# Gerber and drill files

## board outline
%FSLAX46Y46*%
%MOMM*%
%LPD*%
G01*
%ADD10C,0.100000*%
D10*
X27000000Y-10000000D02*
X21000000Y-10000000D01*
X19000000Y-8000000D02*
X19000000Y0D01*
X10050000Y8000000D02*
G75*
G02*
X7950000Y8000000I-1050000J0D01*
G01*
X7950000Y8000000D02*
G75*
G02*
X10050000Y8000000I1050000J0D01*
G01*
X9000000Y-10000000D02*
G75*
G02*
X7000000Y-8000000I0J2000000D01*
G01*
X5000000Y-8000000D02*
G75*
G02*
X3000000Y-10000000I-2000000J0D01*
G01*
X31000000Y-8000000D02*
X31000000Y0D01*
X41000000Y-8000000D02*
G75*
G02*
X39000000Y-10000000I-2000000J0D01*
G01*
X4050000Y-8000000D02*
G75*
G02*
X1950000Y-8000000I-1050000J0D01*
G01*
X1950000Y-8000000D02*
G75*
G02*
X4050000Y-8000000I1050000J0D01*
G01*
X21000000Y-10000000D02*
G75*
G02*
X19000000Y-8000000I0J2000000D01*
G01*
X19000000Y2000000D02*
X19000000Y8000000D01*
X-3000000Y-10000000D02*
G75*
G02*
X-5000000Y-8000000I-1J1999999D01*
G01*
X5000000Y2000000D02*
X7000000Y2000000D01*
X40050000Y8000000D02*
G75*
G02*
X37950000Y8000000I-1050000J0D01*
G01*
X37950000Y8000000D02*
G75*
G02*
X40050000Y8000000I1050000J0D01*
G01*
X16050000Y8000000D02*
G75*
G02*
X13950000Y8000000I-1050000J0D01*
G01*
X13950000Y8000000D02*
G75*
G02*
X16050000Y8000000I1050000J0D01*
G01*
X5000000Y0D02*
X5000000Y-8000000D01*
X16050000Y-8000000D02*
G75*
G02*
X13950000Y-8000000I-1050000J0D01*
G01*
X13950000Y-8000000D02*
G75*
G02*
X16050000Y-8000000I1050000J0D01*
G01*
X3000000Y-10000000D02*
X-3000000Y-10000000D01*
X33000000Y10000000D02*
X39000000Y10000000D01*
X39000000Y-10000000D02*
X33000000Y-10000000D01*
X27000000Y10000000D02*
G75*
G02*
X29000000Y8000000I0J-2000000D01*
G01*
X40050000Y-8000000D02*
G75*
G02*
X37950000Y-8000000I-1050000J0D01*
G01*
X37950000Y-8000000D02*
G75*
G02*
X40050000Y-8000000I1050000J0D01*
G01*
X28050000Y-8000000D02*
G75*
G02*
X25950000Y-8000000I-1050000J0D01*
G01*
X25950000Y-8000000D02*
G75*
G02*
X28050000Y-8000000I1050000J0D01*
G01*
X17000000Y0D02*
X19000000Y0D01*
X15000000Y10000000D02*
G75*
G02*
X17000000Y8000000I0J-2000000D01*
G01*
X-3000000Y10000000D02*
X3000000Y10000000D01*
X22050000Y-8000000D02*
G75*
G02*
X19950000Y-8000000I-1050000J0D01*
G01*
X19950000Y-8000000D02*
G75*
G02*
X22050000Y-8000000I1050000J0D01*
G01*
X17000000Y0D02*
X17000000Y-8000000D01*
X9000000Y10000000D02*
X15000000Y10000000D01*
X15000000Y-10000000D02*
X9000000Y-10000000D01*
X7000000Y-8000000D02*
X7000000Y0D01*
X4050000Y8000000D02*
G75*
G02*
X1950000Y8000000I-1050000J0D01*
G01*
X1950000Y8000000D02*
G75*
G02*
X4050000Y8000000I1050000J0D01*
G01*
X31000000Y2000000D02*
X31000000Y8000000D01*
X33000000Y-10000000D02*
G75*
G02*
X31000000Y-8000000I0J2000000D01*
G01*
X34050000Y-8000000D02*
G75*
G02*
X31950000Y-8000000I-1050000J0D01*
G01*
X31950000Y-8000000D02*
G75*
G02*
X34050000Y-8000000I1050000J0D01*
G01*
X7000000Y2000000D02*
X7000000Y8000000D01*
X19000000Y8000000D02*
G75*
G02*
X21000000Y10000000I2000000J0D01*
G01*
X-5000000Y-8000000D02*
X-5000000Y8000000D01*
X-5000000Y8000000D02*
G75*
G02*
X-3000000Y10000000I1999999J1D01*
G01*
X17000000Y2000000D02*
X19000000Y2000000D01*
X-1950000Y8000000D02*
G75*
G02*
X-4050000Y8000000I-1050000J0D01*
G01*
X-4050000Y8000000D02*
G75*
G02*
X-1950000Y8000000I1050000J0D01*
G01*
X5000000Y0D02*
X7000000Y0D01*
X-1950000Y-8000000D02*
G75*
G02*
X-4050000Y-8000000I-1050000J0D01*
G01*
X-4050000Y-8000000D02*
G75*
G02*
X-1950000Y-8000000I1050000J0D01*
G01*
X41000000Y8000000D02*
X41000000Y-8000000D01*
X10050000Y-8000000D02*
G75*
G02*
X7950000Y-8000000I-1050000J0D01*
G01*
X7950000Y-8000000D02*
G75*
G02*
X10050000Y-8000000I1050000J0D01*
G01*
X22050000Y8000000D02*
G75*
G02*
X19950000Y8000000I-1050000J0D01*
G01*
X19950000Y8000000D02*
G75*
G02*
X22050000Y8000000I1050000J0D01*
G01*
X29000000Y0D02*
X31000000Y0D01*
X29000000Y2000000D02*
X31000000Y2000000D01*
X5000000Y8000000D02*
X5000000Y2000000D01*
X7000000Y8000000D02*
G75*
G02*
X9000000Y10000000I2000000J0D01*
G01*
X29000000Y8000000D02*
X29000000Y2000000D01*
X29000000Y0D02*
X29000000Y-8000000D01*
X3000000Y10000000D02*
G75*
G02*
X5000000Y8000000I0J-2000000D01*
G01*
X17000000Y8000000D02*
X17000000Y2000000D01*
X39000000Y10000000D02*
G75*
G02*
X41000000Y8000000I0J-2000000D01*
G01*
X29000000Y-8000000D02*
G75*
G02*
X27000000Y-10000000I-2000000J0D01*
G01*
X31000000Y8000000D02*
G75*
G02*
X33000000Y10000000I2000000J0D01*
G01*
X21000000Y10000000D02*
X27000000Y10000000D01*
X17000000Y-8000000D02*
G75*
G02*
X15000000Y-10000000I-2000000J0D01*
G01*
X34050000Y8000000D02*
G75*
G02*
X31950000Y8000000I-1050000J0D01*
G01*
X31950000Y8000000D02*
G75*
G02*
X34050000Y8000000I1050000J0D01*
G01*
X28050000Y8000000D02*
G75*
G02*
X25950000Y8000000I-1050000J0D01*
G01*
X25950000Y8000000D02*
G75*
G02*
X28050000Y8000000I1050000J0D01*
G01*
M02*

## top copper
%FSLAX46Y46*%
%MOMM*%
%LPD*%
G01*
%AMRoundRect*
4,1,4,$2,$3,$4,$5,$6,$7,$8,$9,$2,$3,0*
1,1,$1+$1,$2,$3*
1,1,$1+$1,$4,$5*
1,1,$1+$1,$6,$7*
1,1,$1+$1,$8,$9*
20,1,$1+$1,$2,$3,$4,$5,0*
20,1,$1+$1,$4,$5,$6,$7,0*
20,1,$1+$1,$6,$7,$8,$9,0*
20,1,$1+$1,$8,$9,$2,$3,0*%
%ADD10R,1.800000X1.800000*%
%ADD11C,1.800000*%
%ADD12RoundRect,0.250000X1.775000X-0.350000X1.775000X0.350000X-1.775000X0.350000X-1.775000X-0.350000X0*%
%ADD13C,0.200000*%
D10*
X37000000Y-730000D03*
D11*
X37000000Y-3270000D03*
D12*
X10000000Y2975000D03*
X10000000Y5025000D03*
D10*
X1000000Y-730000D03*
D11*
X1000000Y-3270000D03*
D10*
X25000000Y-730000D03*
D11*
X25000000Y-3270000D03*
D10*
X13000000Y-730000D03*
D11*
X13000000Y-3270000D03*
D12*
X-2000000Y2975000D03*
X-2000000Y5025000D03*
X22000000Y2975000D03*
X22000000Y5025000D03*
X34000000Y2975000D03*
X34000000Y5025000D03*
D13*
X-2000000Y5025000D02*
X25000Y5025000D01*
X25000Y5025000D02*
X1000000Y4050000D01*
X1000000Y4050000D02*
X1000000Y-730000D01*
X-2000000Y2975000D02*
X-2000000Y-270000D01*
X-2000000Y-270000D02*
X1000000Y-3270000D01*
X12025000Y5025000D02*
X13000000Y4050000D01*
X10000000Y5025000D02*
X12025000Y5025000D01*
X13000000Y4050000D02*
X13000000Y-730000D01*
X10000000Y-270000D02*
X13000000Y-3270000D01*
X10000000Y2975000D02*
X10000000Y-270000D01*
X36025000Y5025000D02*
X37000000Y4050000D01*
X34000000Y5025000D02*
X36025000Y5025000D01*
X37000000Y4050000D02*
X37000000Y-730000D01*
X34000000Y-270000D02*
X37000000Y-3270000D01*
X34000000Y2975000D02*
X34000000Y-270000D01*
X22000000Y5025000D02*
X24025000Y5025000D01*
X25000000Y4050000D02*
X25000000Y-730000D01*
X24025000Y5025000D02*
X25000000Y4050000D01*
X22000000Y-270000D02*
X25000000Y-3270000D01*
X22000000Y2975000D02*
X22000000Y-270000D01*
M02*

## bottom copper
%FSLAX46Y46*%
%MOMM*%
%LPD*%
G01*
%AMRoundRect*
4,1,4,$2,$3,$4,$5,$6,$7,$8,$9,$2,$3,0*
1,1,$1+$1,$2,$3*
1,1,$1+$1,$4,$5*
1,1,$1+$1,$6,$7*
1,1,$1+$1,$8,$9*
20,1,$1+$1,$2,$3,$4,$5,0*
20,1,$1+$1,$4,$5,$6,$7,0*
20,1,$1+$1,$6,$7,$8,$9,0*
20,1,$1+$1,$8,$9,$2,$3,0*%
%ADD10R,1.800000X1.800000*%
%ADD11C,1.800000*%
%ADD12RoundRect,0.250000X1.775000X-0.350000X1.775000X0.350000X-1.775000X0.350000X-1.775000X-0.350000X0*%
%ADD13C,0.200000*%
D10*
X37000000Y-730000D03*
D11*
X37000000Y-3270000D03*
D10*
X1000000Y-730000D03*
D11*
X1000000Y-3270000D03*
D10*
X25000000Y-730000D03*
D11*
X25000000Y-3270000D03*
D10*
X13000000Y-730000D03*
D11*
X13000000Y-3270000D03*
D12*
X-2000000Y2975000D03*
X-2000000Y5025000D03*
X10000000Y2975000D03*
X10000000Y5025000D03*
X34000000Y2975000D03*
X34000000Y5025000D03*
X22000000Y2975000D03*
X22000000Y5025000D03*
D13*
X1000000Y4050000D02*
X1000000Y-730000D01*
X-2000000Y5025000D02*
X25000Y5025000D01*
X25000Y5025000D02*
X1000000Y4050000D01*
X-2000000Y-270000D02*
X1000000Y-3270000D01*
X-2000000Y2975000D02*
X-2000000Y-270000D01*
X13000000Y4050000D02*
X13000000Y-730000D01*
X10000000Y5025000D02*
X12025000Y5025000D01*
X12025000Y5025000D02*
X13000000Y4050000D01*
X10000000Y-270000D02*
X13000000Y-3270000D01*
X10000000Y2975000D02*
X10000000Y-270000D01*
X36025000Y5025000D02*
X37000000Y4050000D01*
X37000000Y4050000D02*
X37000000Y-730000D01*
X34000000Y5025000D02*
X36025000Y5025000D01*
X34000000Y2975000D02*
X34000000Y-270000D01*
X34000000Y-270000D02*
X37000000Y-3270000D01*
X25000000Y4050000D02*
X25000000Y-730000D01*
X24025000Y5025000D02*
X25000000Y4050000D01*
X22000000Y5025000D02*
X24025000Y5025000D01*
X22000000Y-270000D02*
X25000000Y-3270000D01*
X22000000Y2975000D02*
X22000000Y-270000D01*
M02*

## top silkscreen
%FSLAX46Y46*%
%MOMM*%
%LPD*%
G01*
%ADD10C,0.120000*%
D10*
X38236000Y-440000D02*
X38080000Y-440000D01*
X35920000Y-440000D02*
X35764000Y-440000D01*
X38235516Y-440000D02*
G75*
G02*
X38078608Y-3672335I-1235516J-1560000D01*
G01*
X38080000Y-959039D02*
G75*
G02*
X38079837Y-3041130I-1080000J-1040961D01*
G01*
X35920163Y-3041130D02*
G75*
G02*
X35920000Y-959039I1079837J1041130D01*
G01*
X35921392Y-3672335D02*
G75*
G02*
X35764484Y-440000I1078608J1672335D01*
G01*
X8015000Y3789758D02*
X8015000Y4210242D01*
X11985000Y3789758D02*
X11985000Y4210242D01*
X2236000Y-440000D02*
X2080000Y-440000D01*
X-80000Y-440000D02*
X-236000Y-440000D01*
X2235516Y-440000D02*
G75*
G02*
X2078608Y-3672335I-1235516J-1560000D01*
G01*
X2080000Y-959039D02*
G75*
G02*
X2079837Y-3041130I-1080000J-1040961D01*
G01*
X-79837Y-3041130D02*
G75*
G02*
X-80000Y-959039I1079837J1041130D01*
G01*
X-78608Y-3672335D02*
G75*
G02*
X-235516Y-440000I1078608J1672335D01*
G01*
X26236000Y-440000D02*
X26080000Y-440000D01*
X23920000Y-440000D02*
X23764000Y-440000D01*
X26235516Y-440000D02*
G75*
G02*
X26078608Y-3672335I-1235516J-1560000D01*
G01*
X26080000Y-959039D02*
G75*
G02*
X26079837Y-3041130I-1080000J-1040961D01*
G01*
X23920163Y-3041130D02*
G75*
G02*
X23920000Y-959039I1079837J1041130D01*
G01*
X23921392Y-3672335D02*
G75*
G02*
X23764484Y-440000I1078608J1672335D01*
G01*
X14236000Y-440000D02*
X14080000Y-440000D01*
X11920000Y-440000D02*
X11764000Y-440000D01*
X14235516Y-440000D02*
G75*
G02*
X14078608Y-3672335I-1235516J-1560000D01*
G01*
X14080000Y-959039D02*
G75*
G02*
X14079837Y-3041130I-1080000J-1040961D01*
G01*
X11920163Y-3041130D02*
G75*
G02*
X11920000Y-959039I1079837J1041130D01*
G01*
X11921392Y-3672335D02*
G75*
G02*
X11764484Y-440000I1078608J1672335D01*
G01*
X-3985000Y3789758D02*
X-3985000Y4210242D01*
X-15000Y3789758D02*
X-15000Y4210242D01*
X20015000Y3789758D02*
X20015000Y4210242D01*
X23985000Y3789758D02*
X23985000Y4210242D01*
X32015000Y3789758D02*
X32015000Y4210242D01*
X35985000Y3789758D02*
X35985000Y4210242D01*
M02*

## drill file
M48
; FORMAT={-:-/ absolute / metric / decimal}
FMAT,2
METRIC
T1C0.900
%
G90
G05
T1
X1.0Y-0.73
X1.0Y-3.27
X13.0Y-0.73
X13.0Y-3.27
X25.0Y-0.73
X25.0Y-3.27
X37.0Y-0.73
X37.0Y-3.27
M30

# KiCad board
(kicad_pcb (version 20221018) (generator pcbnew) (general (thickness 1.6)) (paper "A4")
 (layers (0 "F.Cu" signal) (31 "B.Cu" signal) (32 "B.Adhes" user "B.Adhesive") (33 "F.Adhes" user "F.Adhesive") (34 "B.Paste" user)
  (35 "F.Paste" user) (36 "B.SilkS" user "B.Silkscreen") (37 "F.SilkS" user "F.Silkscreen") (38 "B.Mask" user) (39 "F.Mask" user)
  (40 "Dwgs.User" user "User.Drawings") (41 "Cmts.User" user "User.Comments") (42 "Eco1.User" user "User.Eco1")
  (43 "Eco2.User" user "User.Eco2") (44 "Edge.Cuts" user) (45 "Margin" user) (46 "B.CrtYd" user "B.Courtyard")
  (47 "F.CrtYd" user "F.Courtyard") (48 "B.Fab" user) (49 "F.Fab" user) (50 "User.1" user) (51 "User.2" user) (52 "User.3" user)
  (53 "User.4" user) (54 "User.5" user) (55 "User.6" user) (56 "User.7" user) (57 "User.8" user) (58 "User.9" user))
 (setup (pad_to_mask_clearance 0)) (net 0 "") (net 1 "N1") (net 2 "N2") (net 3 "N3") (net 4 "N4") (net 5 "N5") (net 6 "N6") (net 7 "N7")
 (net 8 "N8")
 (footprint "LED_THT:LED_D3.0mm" (layer "F.Cu") (at 37 0.73 -90)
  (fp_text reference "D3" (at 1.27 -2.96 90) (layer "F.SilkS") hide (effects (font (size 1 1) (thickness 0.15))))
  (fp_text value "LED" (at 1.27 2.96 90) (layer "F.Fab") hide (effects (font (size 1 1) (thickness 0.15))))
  (fp_line (start -0.29 -1.236) (end -0.29 -1.08) (stroke (width 0.12) (type solid)) (layer "F.SilkS"))
  (fp_line (start -0.29 1.08) (end -0.29 1.236) (stroke (width 0.12) (type solid)) (layer "F.SilkS"))
  (fp_arc (start -0.29 -1.235516) (mid 1.366487 -1.987659) (end 2.942335 -1.078608) (stroke (width 0.12) (type solid)) (layer "F.SilkS"))
  (fp_arc (start 0.229039 -1.08) (mid 1.270117 -1.5) (end 2.31113 -1.079837) (stroke (width 0.12) (type solid)) (layer "F.SilkS"))
  (fp_arc (start 2.31113 1.079837) (mid 1.270117 1.5) (end 0.229039 1.08) (stroke (width 0.12) (type solid)) (layer "F.SilkS"))
  (fp_arc (start 2.942335 1.078608) (mid 1.366487 1.987659) (end -0.29 1.235516) (stroke (width 0.12) (type solid)) (layer "F.SilkS"))
  (pad "1" thru_hole rect (at 0 0 270) (size 1.8 1.8) (drill 0.9) (layers "*.Cu" "*.Mask") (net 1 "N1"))
  (pad "2" thru_hole circle (at 2.54 0 270) (size 1.8 1.8) (drill 0.9) (layers "*.Cu" "*.Mask") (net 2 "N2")))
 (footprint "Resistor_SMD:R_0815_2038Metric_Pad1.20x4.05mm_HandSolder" (layer "F.Cu") (at 10 -4 90)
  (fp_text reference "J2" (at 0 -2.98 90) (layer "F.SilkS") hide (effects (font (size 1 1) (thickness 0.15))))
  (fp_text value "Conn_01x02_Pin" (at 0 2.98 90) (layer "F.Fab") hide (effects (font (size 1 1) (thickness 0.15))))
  (fp_line (start -0.210242 -1.985) (end 0.210242 -1.985) (stroke (width 0.12) (type solid)) (layer "F.SilkS"))
  (fp_line (start -0.210242 1.985) (end 0.210242 1.985) (stroke (width 0.12) (type solid)) (layer "F.SilkS"))
  (pad "1" smd roundrect (at -1.025 0 90) (size 1.2 4.05) (layers "F.Cu" "F.Paste" "F.Mask") (roundrect_rratio 0.2083333333) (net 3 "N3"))
  (pad "2" smd roundrect (at 1.025 0 90) (size 1.2 4.05) (layers "F.Cu" "F.Paste" "F.Mask") (roundrect_rratio 0.2083333333) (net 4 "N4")))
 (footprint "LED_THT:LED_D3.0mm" (layer "F.Cu") (at 1 0.73 -90)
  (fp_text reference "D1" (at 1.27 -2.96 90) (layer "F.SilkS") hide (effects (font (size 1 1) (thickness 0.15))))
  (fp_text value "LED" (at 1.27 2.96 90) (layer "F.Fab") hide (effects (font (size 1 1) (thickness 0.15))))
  (fp_line (start -0.29 -1.236) (end -0.29 -1.08) (stroke (width 0.12) (type solid)) (layer "F.SilkS"))
  (fp_line (start -0.29 1.08) (end -0.29 1.236) (stroke (width 0.12) (type solid)) (layer "F.SilkS"))
  (fp_arc (start -0.29 -1.235516) (mid 1.366487 -1.987659) (end 2.942335 -1.078608) (stroke (width 0.12) (type solid)) (layer "F.SilkS"))
  (fp_arc (start 0.229039 -1.08) (mid 1.270117 -1.5) (end 2.31113 -1.079837) (stroke (width 0.12) (type solid)) (layer "F.SilkS"))
  (fp_arc (start 2.31113 1.079837) (mid 1.270117 1.5) (end 0.229039 1.08) (stroke (width 0.12) (type solid)) (layer "F.SilkS"))
  (fp_arc (start 2.942335 1.078608) (mid 1.366487 1.987659) (end -0.29 1.235516) (stroke (width 0.12) (type solid)) (layer "F.SilkS"))
  (pad "1" thru_hole rect (at 0 0 270) (size 1.8 1.8) (drill 0.9) (layers "*.Cu" "*.Mask") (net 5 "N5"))
  (pad "2" thru_hole circle (at 2.54 0 270) (size 1.8 1.8) (drill 0.9) (layers "*.Cu" "*.Mask") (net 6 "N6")))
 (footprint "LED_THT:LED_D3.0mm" (layer "F.Cu") (at 25 0.73 -90)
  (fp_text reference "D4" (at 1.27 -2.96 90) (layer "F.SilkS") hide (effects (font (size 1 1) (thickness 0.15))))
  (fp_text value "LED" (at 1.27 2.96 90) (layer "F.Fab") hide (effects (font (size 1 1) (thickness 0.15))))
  (fp_line (start -0.29 -1.236) (end -0.29 -1.08) (stroke (width 0.12) (type solid)) (layer "F.SilkS"))
  (fp_line (start -0.29 1.08) (end -0.29 1.236) (stroke (width 0.12) (type solid)) (layer "F.SilkS"))
  (fp_arc (start -0.29 -1.235516) (mid 1.366487 -1.987659) (end 2.942335 -1.078608) (stroke (width 0.12) (type solid)) (layer "F.SilkS"))
  (fp_arc (start 0.229039 -1.08) (mid 1.270117 -1.5) (end 2.31113 -1.079837) (stroke (width 0.12) (type solid)) (layer "F.SilkS"))
  (fp_arc (start 2.31113 1.079837) (mid 1.270117 1.5) (end 0.229039 1.08) (stroke (width 0.12) (type solid)) (layer "F.SilkS"))
  (fp_arc (start 2.942335 1.078608) (mid 1.366487 1.987659) (end -0.29 1.235516) (stroke (width 0.12) (type solid)) (layer "F.SilkS"))
  (pad "1" thru_hole rect (at 0 0 270) (size 1.8 1.8) (drill 0.9) (layers "*.Cu" "*.Mask") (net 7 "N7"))
  (pad "2" thru_hole circle (at 2.54 0 270) (size 1.8 1.8) (drill 0.9) (layers "*.Cu" "*.Mask") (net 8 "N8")))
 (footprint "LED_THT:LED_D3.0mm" (layer "F.Cu") (at 13 0.73 -90)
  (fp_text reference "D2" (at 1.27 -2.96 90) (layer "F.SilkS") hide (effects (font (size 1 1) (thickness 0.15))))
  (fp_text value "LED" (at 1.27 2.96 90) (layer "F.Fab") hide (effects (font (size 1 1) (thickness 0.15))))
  (fp_line (start -0.29 -1.236) (end -0.29 -1.08) (stroke (width 0.12) (type solid)) (layer "F.SilkS"))
  (fp_line (start -0.29 1.08) (end -0.29 1.236) (stroke (width 0.12) (type solid)) (layer "F.SilkS"))
  (fp_arc (start -0.29 -1.235516) (mid 1.366487 -1.987659) (end 2.942335 -1.078608) (stroke (width 0.12) (type solid)) (layer "F.SilkS"))
  (fp_arc (start 0.229039 -1.08) (mid 1.270117 -1.5) (end 2.31113 -1.079837) (stroke (width 0.12) (type solid)) (layer "F.SilkS"))
  (fp_arc (start 2.31113 1.079837) (mid 1.270117 1.5) (end 0.229039 1.08) (stroke (width 0.12) (type solid)) (layer "F.SilkS"))
  (fp_arc (start 2.942335 1.078608) (mid 1.366487 1.987659) (end -0.29 1.235516) (stroke (width 0.12) (type solid)) (layer "F.SilkS"))
  (pad "1" thru_hole rect (at 0 0 270) (size 1.8 1.8) (drill 0.9) (layers "*.Cu" "*.Mask") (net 4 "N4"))
  (pad "2" thru_hole circle (at 2.54 0 270) (size 1.8 1.8) (drill 0.9) (layers "*.Cu" "*.Mask") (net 3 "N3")))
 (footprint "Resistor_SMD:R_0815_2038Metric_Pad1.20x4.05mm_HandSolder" (layer "F.Cu") (at -2 -4 90)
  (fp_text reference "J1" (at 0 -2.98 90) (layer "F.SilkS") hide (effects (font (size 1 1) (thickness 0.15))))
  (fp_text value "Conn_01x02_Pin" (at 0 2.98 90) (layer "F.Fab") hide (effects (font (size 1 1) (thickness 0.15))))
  (fp_line (start -0.210242 -1.985) (end 0.210242 -1.985) (stroke (width 0.12) (type solid)) (layer "F.SilkS"))
  (fp_line (start -0.210242 1.985) (end 0.210242 1.985) (stroke (width 0.12) (type solid)) (layer "F.SilkS"))
  (pad "1" smd roundrect (at -1.025 0 90) (size 1.2 4.05) (layers "F.Cu" "F.Paste" "F.Mask") (roundrect_rratio 0.2083333333) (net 6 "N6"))
  (pad "2" smd roundrect (at 1.025 0 90) (size 1.2 4.05) (layers "F.Cu" "F.Paste" "F.Mask") (roundrect_rratio 0.2083333333) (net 5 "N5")))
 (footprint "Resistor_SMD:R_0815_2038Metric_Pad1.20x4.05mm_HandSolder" (layer "F.Cu") (at 22 -4 90)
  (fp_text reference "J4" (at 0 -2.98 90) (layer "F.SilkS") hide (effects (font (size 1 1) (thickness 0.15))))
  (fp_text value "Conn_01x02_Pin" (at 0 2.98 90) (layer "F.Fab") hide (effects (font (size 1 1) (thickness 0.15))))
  (fp_line (start -0.210242 -1.985) (end 0.210242 -1.985) (stroke (width 0.12) (type solid)) (layer "F.SilkS"))
  (fp_line (start -0.210242 1.985) (end 0.210242 1.985) (stroke (width 0.12) (type solid)) (layer "F.SilkS"))
  (pad "1" smd roundrect (at -1.025 0 90) (size 1.2 4.05) (layers "F.Cu" "F.Paste" "F.Mask") (roundrect_rratio 0.2083333333) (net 8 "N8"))
  (pad "2" smd roundrect (at 1.025 0 90) (size 1.2 4.05) (layers "F.Cu" "F.Paste" "F.Mask") (roundrect_rratio 0.2083333333) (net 7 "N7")))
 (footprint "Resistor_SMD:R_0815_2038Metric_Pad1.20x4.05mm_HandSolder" (layer "F.Cu") (at 34 -4 90)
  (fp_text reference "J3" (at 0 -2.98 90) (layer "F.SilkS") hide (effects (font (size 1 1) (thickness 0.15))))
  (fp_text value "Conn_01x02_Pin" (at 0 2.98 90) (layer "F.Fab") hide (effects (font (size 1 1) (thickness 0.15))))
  (fp_line (start -0.210242 -1.985) (end 0.210242 -1.985) (stroke (width 0.12) (type solid)) (layer "F.SilkS"))
  (fp_line (start -0.210242 1.985) (end 0.210242 1.985) (stroke (width 0.12) (type solid)) (layer "F.SilkS"))
  (pad "1" smd roundrect (at -1.025 0 90) (size 1.2 4.05) (layers "F.Cu" "F.Paste" "F.Mask") (roundrect_rratio 0.2083333333) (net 2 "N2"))
  (pad "2" smd roundrect (at 1.025 0 90) (size 1.2 4.05) (layers "F.Cu" "F.Paste" "F.Mask") (roundrect_rratio 0.2083333333) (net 1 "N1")))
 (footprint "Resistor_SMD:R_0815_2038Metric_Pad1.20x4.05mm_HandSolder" (layer "B.Cu") (at -2 -4 90)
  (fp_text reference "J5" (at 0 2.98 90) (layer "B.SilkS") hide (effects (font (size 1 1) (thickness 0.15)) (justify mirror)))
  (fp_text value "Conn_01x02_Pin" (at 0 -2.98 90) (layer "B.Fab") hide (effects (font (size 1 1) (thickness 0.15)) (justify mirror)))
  (pad "1" smd roundrect (at -1.025 0 90) (size 1.2 4.05) (layers "B.Cu" "B.Paste" "B.Mask") (roundrect_rratio 0.2083333333) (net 6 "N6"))
  (pad "2" smd roundrect (at 1.025 0 90) (size 1.2 4.05) (layers "B.Cu" "B.Paste" "B.Mask") (roundrect_rratio 0.2083333333) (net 5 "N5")))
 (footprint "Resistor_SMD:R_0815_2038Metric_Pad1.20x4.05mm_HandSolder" (layer "B.Cu") (at 10 -4 90)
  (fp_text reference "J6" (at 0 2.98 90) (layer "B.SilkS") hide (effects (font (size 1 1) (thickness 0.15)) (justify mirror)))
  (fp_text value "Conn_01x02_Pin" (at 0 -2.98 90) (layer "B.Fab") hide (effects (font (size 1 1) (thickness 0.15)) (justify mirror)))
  (pad "1" smd roundrect (at -1.025 0 90) (size 1.2 4.05) (layers "B.Cu" "B.Paste" "B.Mask") (roundrect_rratio 0.2083333333) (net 3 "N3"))
  (pad "2" smd roundrect (at 1.025 0 90) (size 1.2 4.05) (layers "B.Cu" "B.Paste" "B.Mask") (roundrect_rratio 0.2083333333) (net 4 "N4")))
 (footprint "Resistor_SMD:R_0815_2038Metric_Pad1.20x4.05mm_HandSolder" (layer "B.Cu") (at 34 -4 90)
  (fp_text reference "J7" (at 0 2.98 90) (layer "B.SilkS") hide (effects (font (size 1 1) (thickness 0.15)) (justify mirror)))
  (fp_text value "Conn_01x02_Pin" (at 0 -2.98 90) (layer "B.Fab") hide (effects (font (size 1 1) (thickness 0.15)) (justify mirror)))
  (pad "1" smd roundrect (at -1.025 0 90) (size 1.2 4.05) (layers "B.Cu" "B.Paste" "B.Mask") (roundrect_rratio 0.2083333333) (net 2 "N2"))
  (pad "2" smd roundrect (at 1.025 0 90) (size 1.2 4.05) (layers "B.Cu" "B.Paste" "B.Mask") (roundrect_rratio 0.2083333333) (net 1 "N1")))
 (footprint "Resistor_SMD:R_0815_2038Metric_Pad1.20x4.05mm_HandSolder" (layer "B.Cu") (at 22 -4 90)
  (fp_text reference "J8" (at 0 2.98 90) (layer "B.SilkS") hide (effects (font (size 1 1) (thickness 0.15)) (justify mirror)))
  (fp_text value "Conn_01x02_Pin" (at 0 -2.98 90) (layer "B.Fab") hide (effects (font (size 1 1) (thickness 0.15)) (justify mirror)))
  (pad "1" smd roundrect (at -1.025 0 90) (size 1.2 4.05) (layers "B.Cu" "B.Paste" "B.Mask") (roundrect_rratio 0.2083333333) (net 8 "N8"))
  (pad "2" smd roundrect (at 1.025 0 90) (size 1.2 4.05) (layers "B.Cu" "B.Paste" "B.Mask") (roundrect_rratio 0.2083333333) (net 7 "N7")))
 (gr_line (start 27 10) (end 21 10) (stroke (width 0.1) (type solid)) (layer "Edge.Cuts"))
 (gr_line (start 19 8) (end 19 0) (stroke (width 0.1) (type solid)) (layer "Edge.Cuts"))
 (gr_circle (center 9 -8) (end 10.05 -8) (stroke (width 0.1) (type solid)) (fill none) (layer "Edge.Cuts"))
 (gr_arc (start 9 10) (mid 7.585786 9.414214) (end 7 8) (stroke (width 0.1) (type solid)) (layer "Edge.Cuts"))
 (gr_arc (start 5 8) (mid 4.414214 9.414214) (end 3 10) (stroke (width 0.1) (type solid)) (layer "Edge.Cuts"))
 (gr_line (start 31 8) (end 31 0) (stroke (width 0.1) (type solid)) (layer "Edge.Cuts"))
 (gr_arc (start 41 8) (mid 40.414214 9.414214) (end 39 10) (stroke (width 0.1) (type solid)) (layer "Edge.Cuts"))
 (gr_circle (center 3 8) (end 4.05 8) (stroke (width 0.1) (type solid)) (fill none) (layer "Edge.Cuts"))
 (gr_arc (start 21 10) (mid 19.585786 9.414214) (end 19 8) (stroke (width 0.1) (type solid)) (layer "Edge.Cuts"))
 (gr_line (start 19 -2) (end 19 -8) (stroke (width 0.1) (type solid)) (layer "Edge.Cuts"))
 (gr_arc (start -3 10) (mid -4.414214 9.414214) (end -5 8) (stroke (width 0.1) (type solid)) (layer "Edge.Cuts"))
 (gr_line (start 5 -2) (end 7 -2) (stroke (width 0.1) (type solid)) (layer "Edge.Cuts"))
 (gr_circle (center 39 -8) (end 40.05 -8) (stroke (width 0.1) (type solid)) (fill none) (layer "Edge.Cuts"))
 (gr_circle (center 15 -8) (end 16.05 -8) (stroke (width 0.1) (type solid)) (fill none) (layer "Edge.Cuts"))
 (gr_line (start 5 0) (end 5 8) (stroke (width 0.1) (type solid)) (layer "Edge.Cuts"))
 (gr_circle (center 15 8) (end 16.05 8) (stroke (width 0.1) (type solid)) (fill none) (layer "Edge.Cuts"))
 (gr_line (start 3 10) (end -3 10) (stroke (width 0.1) (type solid)) (layer "Edge.Cuts"))
 (gr_line (start 33 -10) (end 39 -10) (stroke (width 0.1) (type solid)) (layer "Edge.Cuts"))
 (gr_line (start 39 10) (end 33 10) (stroke (width 0.1) (type solid)) (layer "Edge.Cuts"))
 (gr_arc (start 27 -10) (mid 28.414214 -9.414214) (end 29 -8) (stroke (width 0.1) (type solid)) (layer "Edge.Cuts"))
 (gr_circle (center 39 8) (end 40.05 8) (stroke (width 0.1) (type solid)) (fill none) (layer "Edge.Cuts"))
 (gr_circle (center 27 8) (end 28.05 8) (stroke (width 0.1) (type solid)) (fill none) (layer "Edge.Cuts"))
 (gr_line (start 17 0) (end 19 0) (stroke (width 0.1) (type solid)) (layer "Edge.Cuts"))
 (gr_arc (start 15 -10) (mid 16.414214 -9.414214) (end 17 -8) (stroke (width 0.1) (type solid)) (layer "Edge.Cuts"))
 (gr_line (start -3 -10) (end 3 -10) (stroke (width 0.1) (type solid)) (layer "Edge.Cuts"))
 (gr_circle (center 21 8) (end 22.05 8) (stroke (width 0.1) (type solid)) (fill none) (layer "Edge.Cuts"))
 (gr_line (start 17 0) (end 17 8) (stroke (width 0.1) (type solid)) (layer "Edge.Cuts"))
 (gr_line (start 9 -10) (end 15 -10) (stroke (width 0.1) (type solid)) (layer "Edge.Cuts"))
 (gr_line (start 15 10) (end 9 10) (stroke (width 0.1) (type solid)) (layer "Edge.Cuts"))
 (gr_line (start 7 8) (end 7 0) (stroke (width 0.1) (type solid)) (layer "Edge.Cuts"))
 (gr_circle (center 3 -8) (end 4.05 -8) (stroke (width 0.1) (type solid)) (fill none) (layer "Edge.Cuts"))
 (gr_line (start 31 -2) (end 31 -8) (stroke (width 0.1) (type solid)) (layer "Edge.Cuts"))
 (gr_arc (start 33 10) (mid 31.585786 9.414214) (end 31 8) (stroke (width 0.1) (type solid)) (layer "Edge.Cuts"))
 (gr_circle (center 33 8) (end 34.05 8) (stroke (width 0.1) (type solid)) (fill none) (layer "Edge.Cuts"))
 (gr_line (start 7 -2) (end 7 -8) (stroke (width 0.1) (type solid)) (layer "Edge.Cuts"))
 (gr_arc (start 19 -8) (mid 19.585786 -9.414214) (end 21 -10) (stroke (width 0.1) (type solid)) (layer "Edge.Cuts"))
 (gr_line (start -5 8) (end -5 -8) (stroke (width 0.1) (type solid)) (layer "Edge.Cuts"))
 (gr_arc (start -5 -8) (mid -4.414214 -9.414214) (end -3 -10) (stroke (width 0.1) (type solid)) (layer "Edge.Cuts"))
 (gr_line (start 17 -2) (end 19 -2) (stroke (width 0.1) (type solid)) (layer "Edge.Cuts"))
 (gr_circle (center -3 -8) (end -1.95 -8) (stroke (width 0.1) (type solid)) (fill none) (layer "Edge.Cuts"))
 (gr_line (start 5 0) (end 7 0) (stroke (width 0.1) (type solid)) (layer "Edge.Cuts"))
 (gr_circle (center -3 8) (end -1.95 8) (stroke (width 0.1) (type solid)) (fill none) (layer "Edge.Cuts"))
 (gr_line (start 41 -8) (end 41 8) (stroke (width 0.1) (type solid)) (layer "Edge.Cuts"))
 (gr_circle (center 9 8) (end 10.05 8) (stroke (width 0.1) (type solid)) (fill none) (layer "Edge.Cuts"))
 (gr_circle (center 21 -8) (end 22.05 -8) (stroke (width 0.1) (type solid)) (fill none) (layer "Edge.Cuts"))
 (gr_line (start 29 0) (end 31 0) (stroke (width 0.1) (type solid)) (layer "Edge.Cuts"))
 (gr_line (start 29 -2) (end 31 -2) (stroke (width 0.1) (type solid)) (layer "Edge.Cuts"))
 (gr_line (start 5 -8) (end 5 -2) (stroke (width 0.1) (type solid)) (layer "Edge.Cuts"))
 (gr_arc (start 7 -8) (mid 7.585786 -9.414214) (end 9 -10) (stroke (width 0.1) (type solid)) (layer "Edge.Cuts"))
 (gr_line (start 29 -8) (end 29 -2) (stroke (width 0.1) (type solid)) (layer "Edge.Cuts"))
 (gr_line (start 29 0) (end 29 8) (stroke (width 0.1) (type solid)) (layer "Edge.Cuts"))
 (gr_arc (start 3 -10) (mid 4.414214 -9.414214) (end 5 -8) (stroke (width 0.1) (type solid)) (layer "Edge.Cuts"))
 (gr_line (start 17 -8) (end 17 -2) (stroke (width 0.1) (type solid)) (layer "Edge.Cuts"))
 (gr_arc (start 39 -10) (mid 40.414214 -9.414214) (end 41 -8) (stroke (width 0.1) (type solid)) (layer "Edge.Cuts"))
 (gr_arc (start 29 8) (mid 28.414214 9.414214) (end 27 10) (stroke (width 0.1) (type solid)) (layer "Edge.Cuts"))
 (gr_arc (start 31 -8) (mid 31.585786 -9.414214) (end 33 -10) (stroke (width 0.1) (type solid)) (layer "Edge.Cuts"))
 (gr_line (start 21 -10) (end 27 -10) (stroke (width 0.1) (type solid)) (layer "Edge.Cuts"))
 (gr_arc (start 17 8) (mid 16.414214 9.414214) (end 15 10) (stroke (width 0.1) (type solid)) (layer "Edge.Cuts"))
 (gr_circle (center 33 -8) (end 34.05 -8) (stroke (width 0.1) (type solid)) (fill none) (layer "Edge.Cuts"))
 (gr_circle (center 27 -8) (end 28.05 -8) (stroke (width 0.1) (type solid)) (fill none) (layer "Edge.Cuts"))
 (segment (start -2 -5.025) (end 0.025 -5.025) (width 0.2) (layer "F.Cu") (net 5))
 (segment (start 0.025 -5.025) (end 1 -4.05) (width 0.2) (layer "F.Cu") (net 5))
 (segment (start 1 -4.05) (end 1 0.73) (width 0.2) (layer "F.Cu") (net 5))
 (segment (start 1 -4.05) (end 1 0.73) (width 0.2) (layer "B.Cu") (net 5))
 (segment (start -2 -5.025) (end 0.025 -5.025) (width 0.2) (layer "B.Cu") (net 5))
 (segment (start 0.025 -5.025) (end 1 -4.05) (width 0.2) (layer "B.Cu") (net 5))
 (segment (start -2 -2.975) (end -2 0.27) (width 0.2) (layer "F.Cu") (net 6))
 (segment (start -2 0.27) (end 1 3.27) (width 0.2) (layer "F.Cu") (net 6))
 (segment (start -2 0.27) (end 1 3.27) (width 0.2) (layer "B.Cu") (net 6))
 (segment (start -2 -2.975) (end -2 0.27) (width 0.2) (layer "B.Cu") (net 6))
 (segment (start 12.025 -5.025) (end 13 -4.05) (width 0.2) (layer "F.Cu") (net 4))
 (segment (start 10 -5.025) (end 12.025 -5.025) (width 0.2) (layer "F.Cu") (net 4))
 (segment (start 13 -4.05) (end 13 0.73) (width 0.2) (layer "F.Cu") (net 4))
 (segment (start 13 -4.05) (end 13 0.73) (width 0.2) (layer "B.Cu") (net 4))
 (segment (start 10 -5.025) (end 12.025 -5.025) (width 0.2) (layer "B.Cu") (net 4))
 (segment (start 12.025 -5.025) (end 13 -4.05) (width 0.2) (layer "B.Cu") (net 4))
 (segment (start 10 0.27) (end 13 3.27) (width 0.2) (layer "F.Cu") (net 3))
 (segment (start 10 -2.975) (end 10 0.27) (width 0.2) (layer "F.Cu") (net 3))
 (segment (start 10 0.27) (end 13 3.27) (width 0.2) (layer "B.Cu") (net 3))
 (segment (start 10 -2.975) (end 10 0.27) (width 0.2) (layer "B.Cu") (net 3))
 (segment (start 36.025 -5.025) (end 37 -4.05) (width 0.2) (layer "F.Cu") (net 1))
 (segment (start 34 -5.025) (end 36.025 -5.025) (width 0.2) (layer "F.Cu") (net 1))
 (segment (start 37 -4.05) (end 37 0.73) (width 0.2) (layer "F.Cu") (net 1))
 (segment (start 36.025 -5.025) (end 37 -4.05) (width 0.2) (layer "B.Cu") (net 1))
 (segment (start 37 -4.05) (end 37 0.73) (width 0.2) (layer "B.Cu") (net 1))
 (segment (start 34 -5.025) (end 36.025 -5.025) (width 0.2) (layer "B.Cu") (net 1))
 (segment (start 34 0.27) (end 37 3.27) (width 0.2) (layer "F.Cu") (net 2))
 (segment (start 34 -2.975) (end 34 0.27) (width 0.2) (layer "F.Cu") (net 2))
 (segment (start 34 -2.975) (end 34 0.27) (width 0.2) (layer "B.Cu") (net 2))
 (segment (start 34 0.27) (end 37 3.27) (width 0.2) (layer "B.Cu") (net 2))
 (segment (start 22 -5.025) (end 24.025 -5.025) (width 0.2) (layer "F.Cu") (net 7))
 (segment (start 25 -4.05) (end 25 0.73) (width 0.2) (layer "F.Cu") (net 7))
 (segment (start 24.025 -5.025) (end 25 -4.05) (width 0.2) (layer "F.Cu") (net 7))
 (segment (start 25 -4.05) (end 25 0.73) (width 0.2) (layer "B.Cu") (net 7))
 (segment (start 24.025 -5.025) (end 25 -4.05) (width 0.2) (layer "B.Cu") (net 7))
 (segment (start 22 -5.025) (end 24.025 -5.025) (width 0.2) (layer "B.Cu") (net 7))
 (segment (start 22 0.27) (end 25 3.27) (width 0.2) (layer "F.Cu") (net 8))
 (segment (start 22 -2.975) (end 22 0.27) (width 0.2) (layer "F.Cu") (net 8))
 (segment (start 22 0.27) (end 25 3.27) (width 0.2) (layer "B.Cu") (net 8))
 (segment (start 22 -2.975) (end 22 0.27) (width 0.2) (layer "B.Cu") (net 8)))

